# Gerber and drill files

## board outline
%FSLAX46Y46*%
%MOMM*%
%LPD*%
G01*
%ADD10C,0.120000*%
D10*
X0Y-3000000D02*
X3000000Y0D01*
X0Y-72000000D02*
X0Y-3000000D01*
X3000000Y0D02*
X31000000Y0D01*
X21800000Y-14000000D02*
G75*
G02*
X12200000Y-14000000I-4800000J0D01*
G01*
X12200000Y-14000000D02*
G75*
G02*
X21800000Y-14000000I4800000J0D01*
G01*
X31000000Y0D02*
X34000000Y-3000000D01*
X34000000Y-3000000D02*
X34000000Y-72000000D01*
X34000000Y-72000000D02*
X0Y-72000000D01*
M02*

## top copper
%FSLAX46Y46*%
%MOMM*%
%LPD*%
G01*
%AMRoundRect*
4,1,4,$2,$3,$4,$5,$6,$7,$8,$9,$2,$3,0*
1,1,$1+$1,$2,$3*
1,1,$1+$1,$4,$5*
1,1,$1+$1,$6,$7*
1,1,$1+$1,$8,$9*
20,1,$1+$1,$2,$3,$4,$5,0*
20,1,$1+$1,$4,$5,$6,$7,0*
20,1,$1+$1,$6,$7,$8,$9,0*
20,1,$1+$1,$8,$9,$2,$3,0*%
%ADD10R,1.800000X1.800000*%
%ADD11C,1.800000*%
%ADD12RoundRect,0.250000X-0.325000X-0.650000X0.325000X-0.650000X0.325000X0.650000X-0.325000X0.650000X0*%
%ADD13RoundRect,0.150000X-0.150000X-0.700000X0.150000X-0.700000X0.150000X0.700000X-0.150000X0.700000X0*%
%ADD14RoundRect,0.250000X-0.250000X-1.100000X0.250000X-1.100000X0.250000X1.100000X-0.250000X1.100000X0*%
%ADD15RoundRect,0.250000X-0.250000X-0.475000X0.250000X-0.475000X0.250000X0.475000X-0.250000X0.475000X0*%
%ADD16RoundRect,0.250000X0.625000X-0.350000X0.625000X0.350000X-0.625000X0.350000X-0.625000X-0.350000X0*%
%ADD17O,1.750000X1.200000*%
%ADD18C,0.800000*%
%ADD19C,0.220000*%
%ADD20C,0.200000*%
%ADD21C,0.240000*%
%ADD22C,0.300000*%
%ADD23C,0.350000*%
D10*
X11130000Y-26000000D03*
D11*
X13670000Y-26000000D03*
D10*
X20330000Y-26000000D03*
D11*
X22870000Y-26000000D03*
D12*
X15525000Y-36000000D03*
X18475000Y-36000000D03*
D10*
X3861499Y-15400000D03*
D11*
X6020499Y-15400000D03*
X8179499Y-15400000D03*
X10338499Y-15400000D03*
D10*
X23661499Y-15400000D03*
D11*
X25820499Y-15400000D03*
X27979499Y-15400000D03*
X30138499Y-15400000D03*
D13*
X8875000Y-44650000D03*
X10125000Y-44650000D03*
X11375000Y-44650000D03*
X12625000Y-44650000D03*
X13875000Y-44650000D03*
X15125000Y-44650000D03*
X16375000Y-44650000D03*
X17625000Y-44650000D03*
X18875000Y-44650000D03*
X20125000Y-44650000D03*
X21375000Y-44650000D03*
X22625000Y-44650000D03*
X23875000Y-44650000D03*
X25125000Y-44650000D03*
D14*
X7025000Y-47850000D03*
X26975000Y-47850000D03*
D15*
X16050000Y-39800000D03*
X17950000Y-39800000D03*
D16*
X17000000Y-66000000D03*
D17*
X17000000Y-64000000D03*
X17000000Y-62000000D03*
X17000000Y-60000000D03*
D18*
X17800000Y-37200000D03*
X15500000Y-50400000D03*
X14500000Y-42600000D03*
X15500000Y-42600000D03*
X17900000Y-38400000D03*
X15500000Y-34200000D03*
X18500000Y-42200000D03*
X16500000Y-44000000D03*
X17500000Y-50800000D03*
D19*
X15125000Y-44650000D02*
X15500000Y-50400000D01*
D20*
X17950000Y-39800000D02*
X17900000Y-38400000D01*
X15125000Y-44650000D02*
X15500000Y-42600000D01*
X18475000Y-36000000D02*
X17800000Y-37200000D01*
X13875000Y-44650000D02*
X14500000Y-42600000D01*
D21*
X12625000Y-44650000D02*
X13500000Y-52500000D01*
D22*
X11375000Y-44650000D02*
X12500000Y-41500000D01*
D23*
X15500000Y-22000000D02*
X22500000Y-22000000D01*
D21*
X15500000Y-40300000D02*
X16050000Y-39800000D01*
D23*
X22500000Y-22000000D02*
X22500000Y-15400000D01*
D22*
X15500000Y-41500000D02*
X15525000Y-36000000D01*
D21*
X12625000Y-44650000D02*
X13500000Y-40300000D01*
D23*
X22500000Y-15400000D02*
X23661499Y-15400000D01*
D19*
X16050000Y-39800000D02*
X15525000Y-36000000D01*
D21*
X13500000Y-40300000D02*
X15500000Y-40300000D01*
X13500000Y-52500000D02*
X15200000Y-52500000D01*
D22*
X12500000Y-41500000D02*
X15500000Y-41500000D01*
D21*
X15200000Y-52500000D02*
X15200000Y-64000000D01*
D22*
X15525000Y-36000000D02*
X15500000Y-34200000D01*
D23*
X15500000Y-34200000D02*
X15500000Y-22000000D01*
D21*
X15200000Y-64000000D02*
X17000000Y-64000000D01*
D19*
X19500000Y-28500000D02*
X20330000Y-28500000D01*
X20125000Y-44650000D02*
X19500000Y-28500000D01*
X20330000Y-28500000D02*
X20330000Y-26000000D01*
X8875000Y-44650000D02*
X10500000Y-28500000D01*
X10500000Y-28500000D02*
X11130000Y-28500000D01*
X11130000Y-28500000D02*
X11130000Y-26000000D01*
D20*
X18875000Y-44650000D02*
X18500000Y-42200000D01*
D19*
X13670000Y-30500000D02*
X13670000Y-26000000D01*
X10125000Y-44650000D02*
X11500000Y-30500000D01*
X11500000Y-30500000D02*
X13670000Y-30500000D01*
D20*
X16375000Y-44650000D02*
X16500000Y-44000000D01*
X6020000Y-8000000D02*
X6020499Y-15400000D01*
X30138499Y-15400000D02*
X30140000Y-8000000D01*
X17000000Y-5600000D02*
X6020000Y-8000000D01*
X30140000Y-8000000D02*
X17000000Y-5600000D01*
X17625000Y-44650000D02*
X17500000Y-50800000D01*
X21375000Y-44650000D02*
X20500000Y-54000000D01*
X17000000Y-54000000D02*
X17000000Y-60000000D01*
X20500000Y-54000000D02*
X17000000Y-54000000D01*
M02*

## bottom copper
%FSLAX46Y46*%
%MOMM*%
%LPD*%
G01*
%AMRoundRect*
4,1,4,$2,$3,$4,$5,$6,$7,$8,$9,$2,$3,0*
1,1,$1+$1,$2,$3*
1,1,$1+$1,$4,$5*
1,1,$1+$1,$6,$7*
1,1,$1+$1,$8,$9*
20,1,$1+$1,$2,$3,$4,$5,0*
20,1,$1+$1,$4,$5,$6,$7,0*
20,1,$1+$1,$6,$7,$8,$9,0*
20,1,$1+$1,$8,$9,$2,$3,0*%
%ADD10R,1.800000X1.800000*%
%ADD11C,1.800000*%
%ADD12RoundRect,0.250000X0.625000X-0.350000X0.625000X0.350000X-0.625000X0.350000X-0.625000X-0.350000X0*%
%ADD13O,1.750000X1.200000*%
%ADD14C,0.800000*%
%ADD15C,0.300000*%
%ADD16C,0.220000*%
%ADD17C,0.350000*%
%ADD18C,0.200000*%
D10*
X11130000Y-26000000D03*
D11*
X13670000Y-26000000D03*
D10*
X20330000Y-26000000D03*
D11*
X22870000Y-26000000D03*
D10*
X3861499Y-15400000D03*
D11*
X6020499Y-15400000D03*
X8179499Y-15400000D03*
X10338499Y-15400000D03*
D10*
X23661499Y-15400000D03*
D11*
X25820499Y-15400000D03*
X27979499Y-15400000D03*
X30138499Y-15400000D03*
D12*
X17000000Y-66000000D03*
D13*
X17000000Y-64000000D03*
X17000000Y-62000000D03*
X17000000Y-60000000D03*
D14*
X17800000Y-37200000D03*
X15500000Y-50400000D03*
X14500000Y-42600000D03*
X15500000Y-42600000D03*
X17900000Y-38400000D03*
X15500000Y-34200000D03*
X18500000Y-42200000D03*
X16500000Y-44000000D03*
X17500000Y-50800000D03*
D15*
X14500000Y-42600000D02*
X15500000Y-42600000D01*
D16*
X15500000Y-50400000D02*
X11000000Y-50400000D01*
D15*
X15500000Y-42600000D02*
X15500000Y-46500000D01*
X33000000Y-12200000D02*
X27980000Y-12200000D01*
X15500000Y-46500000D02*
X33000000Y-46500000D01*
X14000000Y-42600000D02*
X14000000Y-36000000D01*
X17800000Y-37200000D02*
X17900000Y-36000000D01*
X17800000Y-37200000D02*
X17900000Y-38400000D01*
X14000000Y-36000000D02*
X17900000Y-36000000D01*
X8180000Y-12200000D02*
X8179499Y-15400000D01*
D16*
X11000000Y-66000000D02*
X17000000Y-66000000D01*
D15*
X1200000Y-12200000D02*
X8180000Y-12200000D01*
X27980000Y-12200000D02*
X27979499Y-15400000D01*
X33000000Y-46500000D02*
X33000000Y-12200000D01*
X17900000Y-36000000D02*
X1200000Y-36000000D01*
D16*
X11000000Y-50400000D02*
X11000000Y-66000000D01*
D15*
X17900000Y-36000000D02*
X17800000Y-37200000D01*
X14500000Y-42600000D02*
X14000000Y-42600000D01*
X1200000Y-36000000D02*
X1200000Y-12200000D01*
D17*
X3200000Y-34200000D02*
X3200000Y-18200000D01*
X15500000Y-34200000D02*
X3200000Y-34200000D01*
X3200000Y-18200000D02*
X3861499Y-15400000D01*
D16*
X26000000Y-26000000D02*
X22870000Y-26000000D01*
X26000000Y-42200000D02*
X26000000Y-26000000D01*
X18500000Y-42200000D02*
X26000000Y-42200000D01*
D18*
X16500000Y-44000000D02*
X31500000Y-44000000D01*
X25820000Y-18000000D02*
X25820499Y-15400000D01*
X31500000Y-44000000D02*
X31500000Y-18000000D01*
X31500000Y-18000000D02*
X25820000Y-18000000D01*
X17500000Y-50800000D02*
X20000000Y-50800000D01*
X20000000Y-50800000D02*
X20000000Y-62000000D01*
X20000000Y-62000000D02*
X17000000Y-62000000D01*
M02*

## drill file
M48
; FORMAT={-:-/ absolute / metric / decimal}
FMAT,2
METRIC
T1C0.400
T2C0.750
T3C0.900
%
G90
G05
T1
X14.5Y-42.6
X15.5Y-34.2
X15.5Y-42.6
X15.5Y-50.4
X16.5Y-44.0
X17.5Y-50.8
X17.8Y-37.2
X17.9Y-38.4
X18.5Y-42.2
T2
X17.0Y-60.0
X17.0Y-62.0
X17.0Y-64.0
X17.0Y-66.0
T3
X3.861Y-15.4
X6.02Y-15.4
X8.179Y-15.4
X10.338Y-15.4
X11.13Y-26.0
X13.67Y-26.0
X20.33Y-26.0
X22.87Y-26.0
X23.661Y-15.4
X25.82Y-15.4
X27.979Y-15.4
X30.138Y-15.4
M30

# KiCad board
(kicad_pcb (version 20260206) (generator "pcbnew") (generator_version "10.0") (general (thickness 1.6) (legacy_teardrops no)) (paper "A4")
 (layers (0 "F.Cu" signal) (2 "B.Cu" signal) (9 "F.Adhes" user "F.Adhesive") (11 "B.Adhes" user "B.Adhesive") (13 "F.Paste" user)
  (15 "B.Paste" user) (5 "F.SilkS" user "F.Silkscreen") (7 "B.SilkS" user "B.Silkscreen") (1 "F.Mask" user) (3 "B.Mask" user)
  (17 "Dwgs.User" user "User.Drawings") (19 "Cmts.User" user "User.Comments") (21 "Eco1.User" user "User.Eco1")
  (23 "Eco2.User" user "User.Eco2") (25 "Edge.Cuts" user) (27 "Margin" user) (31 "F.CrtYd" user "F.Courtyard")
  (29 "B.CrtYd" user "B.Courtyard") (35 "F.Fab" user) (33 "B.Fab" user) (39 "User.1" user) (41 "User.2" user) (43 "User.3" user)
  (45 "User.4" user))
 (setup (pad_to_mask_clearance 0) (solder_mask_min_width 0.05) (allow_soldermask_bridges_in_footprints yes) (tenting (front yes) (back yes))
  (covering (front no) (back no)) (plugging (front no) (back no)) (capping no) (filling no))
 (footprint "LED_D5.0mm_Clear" (layer "F.Cu") (at 11.13 26)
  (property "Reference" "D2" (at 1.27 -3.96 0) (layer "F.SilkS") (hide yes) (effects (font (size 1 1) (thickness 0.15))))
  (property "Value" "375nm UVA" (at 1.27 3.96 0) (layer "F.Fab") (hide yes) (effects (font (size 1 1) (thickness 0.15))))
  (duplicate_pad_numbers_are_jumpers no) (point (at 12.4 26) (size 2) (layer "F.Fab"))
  (pad "1" thru_hole rect (at 0 0) (size 1.8 1.8) (drill 0.9) (layers "*.Cu" "*.Mask") (remove_unused_layers no) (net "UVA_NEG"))
  (pad "2" thru_hole circle (at 2.54 0) (size 1.8 1.8) (drill 0.9) (layers "*.Cu" "*.Mask") (remove_unused_layers no) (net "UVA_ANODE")))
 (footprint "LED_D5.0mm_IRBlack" (layer "F.Cu") (at 20.33 26)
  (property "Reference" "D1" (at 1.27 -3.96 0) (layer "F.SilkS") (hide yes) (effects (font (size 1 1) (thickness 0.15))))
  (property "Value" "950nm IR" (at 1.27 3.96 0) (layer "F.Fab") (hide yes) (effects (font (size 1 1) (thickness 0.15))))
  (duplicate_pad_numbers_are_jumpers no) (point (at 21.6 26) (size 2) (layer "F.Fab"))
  (pad "1" thru_hole rect (at 0 0) (size 1.8 1.8) (drill 0.9) (layers "*.Cu" "*.Mask") (remove_unused_layers no) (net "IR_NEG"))
  (pad "2" thru_hole circle (at 2.54 0) (size 1.8 1.8) (drill 0.9) (layers "*.Cu" "*.Mask") (remove_unused_layers no) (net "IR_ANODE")))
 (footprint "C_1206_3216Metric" (layer "F.Cu") (at 17 36)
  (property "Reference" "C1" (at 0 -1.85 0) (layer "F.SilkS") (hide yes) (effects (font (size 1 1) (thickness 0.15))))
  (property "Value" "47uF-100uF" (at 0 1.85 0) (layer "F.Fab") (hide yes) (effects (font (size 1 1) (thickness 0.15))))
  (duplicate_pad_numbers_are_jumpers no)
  (pad "1" smd roundrect (at -1.475 0) (size 1.15 1.8) (layers "F.Cu" "F.Mask" "F.Paste") (roundrect_rratio 0.217391) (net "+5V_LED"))
  (pad "2" smd roundrect (at 1.475 0) (size 1.15 1.8) (layers "F.Cu" "F.Mask" "F.Paste") (roundrect_rratio 0.217391) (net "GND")))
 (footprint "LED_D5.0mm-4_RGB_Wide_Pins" (layer "F.Cu") (at 3.861499 15.4)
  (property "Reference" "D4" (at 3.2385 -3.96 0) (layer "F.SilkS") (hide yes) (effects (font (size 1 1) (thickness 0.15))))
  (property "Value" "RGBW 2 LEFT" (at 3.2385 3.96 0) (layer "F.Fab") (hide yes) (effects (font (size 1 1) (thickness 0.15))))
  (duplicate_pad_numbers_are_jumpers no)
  (pad "1" thru_hole rect (at 0 0) (size 1.8 1.8) (drill 0.9) (layers "*.Cu" "*.Mask") (remove_unused_layers no) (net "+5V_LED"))
  (pad "2" thru_hole circle (at 2.159 0) (size 1.8 1.8) (drill 0.9) (layers "*.Cu" "*.Mask") (remove_unused_layers no) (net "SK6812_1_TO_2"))
  (pad "3" thru_hole circle (at 4.318 0) (size 1.8 1.8) (drill 0.9) (layers "*.Cu" "*.Mask") (remove_unused_layers no) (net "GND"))
  (pad "4" thru_hole circle (at 6.477 0) (size 1.8 1.8) (drill 0.9) (layers "*.Cu" "*.Mask") (remove_unused_layers no)))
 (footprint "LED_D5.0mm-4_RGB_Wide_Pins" (layer "F.Cu") (at 23.661499 15.4)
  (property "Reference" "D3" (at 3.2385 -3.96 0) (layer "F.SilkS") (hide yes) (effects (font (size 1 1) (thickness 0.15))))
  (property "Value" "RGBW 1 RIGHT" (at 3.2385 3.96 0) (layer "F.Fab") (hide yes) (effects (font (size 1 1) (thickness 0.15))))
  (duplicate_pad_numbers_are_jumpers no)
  (pad "1" thru_hole rect (at 0 0) (size 1.8 1.8) (drill 0.9) (layers "*.Cu" "*.Mask") (remove_unused_layers no) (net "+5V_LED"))
  (pad "2" thru_hole circle (at 2.159 0) (size 1.8 1.8) (drill 0.9) (layers "*.Cu" "*.Mask") (remove_unused_layers no) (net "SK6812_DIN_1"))
  (pad "3" thru_hole circle (at 4.318 0) (size 1.8 1.8) (drill 0.9) (layers "*.Cu" "*.Mask") (remove_unused_layers no) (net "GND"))
  (pad "4" thru_hole circle (at 6.477 0) (size 1.8 1.8) (drill 0.9) (layers "*.Cu" "*.Mask") (remove_unused_layers no) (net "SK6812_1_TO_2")))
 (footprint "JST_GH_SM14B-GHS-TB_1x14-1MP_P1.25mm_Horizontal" (layer "F.Cu") (at 17 46.5)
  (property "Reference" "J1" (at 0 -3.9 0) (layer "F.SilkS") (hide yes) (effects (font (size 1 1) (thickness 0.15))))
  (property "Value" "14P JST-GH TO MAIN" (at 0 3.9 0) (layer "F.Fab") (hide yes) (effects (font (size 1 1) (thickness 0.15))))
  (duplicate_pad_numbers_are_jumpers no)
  (pad "1" smd roundrect (at -8.125 -1.85) (size 0.6 1.7) (layers "F.Cu" "F.Mask" "F.Paste") (roundrect_rratio 0.25) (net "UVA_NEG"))
  (pad "2" smd roundrect (at -6.875 -1.85) (size 0.6 1.7) (layers "F.Cu" "F.Mask" "F.Paste") (roundrect_rratio 0.25) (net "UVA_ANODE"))
  (pad "3" smd roundrect (at -5.625 -1.85) (size 0.6 1.7) (layers "F.Cu" "F.Mask" "F.Paste") (roundrect_rratio 0.25) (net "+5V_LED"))
  (pad "4" smd roundrect (at -4.375 -1.85) (size 0.6 1.7) (layers "F.Cu" "F.Mask" "F.Paste") (roundrect_rratio 0.25) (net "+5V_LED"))
  (pad "5" smd roundrect (at -3.125 -1.85) (size 0.6 1.7) (layers "F.Cu" "F.Mask" "F.Paste") (roundrect_rratio 0.25) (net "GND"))
  (pad "6" smd roundrect (at -1.875 -1.85) (size 0.6 1.7) (layers "F.Cu" "F.Mask" "F.Paste") (roundrect_rratio 0.25) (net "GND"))
  (pad "7" smd roundrect (at -0.625 -1.85) (size 0.6 1.7) (layers "F.Cu" "F.Mask" "F.Paste") (roundrect_rratio 0.25) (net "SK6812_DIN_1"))
  (pad "8" smd roundrect (at 0.625 -1.85) (size 0.6 1.7) (layers "F.Cu" "F.Mask" "F.Paste") (roundrect_rratio 0.25) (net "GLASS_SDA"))
  (pad "9" smd roundrect (at 1.875 -1.85) (size 0.6 1.7) (layers "F.Cu" "F.Mask" "F.Paste") (roundrect_rratio 0.25) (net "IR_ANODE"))
  (pad "10" smd roundrect (at 3.125 -1.85) (size 0.6 1.7) (layers "F.Cu" "F.Mask" "F.Paste") (roundrect_rratio 0.25) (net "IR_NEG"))
  (pad "11" smd roundrect (at 4.375 -1.85) (size 0.6 1.7) (layers "F.Cu" "F.Mask" "F.Paste") (roundrect_rratio 0.25) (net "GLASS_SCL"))
  (pad "12" smd roundrect (at 5.625 -1.85) (size 0.6 1.7) (layers "F.Cu" "F.Mask" "F.Paste") (roundrect_rratio 0.25))
  (pad "13" smd roundrect (at 6.875 -1.85) (size 0.6 1.7) (layers "F.Cu" "F.Mask" "F.Paste") (roundrect_rratio 0.25))
  (pad "14" smd roundrect (at 8.125 -1.85) (size 0.6 1.7) (layers "F.Cu" "F.Mask" "F.Paste") (roundrect_rratio 0.25))
  (pad "MP" smd roundrect (at -9.975 1.35) (size 1 2.7) (layers "F.Cu" "F.Mask" "F.Paste") (roundrect_rratio 0.25))
  (pad "MP" smd roundrect (at 9.975 1.35) (size 1 2.7) (layers "F.Cu" "F.Mask" "F.Paste") (roundrect_rratio 0.25)))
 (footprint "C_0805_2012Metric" (layer "F.Cu") (at 17 39.8)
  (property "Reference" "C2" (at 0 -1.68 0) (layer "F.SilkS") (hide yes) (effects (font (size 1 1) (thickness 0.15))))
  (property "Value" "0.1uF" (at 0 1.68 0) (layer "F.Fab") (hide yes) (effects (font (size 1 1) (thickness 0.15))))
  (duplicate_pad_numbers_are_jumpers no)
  (pad "1" smd roundrect (at -0.95 0) (size 1 1.45) (layers "F.Cu" "F.Mask" "F.Paste") (roundrect_rratio 0.25) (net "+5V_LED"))
  (pad "2" smd roundrect (at 0.95 0) (size 1 1.45) (layers "F.Cu" "F.Mask" "F.Paste") (roundrect_rratio 0.25) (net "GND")))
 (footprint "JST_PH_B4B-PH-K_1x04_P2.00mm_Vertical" (layer "F.Cu") (at 17 66 90)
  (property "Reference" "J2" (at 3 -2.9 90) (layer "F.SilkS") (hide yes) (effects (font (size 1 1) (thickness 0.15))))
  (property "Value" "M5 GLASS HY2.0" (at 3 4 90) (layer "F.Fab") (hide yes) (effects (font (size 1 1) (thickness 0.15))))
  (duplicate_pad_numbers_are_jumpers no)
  (pad "1" thru_hole roundrect (at 0 0 90) (size 1.2 1.75) (drill 0.75) (layers "*.Cu" "*.Mask") (remove_unused_layers no)
   (roundrect_rratio 0.208333) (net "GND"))
  (pad "2" thru_hole oval (at 2 0 90) (size 1.2 1.75) (drill 0.75) (layers "*.Cu" "*.Mask") (remove_unused_layers no) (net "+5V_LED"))
  (pad "3" thru_hole oval (at 4 0 90) (size 1.2 1.75) (drill 0.75) (layers "*.Cu" "*.Mask") (remove_unused_layers no) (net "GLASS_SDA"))
  (pad "4" thru_hole oval (at 6 0 90) (size 1.2 1.75) (drill 0.75) (layers "*.Cu" "*.Mask") (remove_unused_layers no) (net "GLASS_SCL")))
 (gr_line (start 0 3) (end 3 0) (stroke (width 0.12) (type default)) (layer "Edge.Cuts"))
 (gr_line (start 0 72) (end 0 3) (stroke (width 0.12) (type default)) (layer "Edge.Cuts"))
 (gr_line (start 3 0) (end 31 0) (stroke (width 0.12) (type default)) (layer "Edge.Cuts"))
 (gr_circle (center 17 14) (end 21.8 14) (stroke (width 0.12) (type default)) (fill no) (layer "Edge.Cuts"))
 (gr_line (start 31 0) (end 34 3) (stroke (width 0.12) (type default)) (layer "Edge.Cuts"))
 (gr_line (start 34 3) (end 34 72) (stroke (width 0.12) (type default)) (layer "Edge.Cuts"))
 (gr_line (start 34 72) (end 0 72) (stroke (width 0.12) (type default)) (layer "Edge.Cuts"))
 (segment (start 15.125 44.65) (end 15.5 50.4) (width 0.22) (layer "F.Cu") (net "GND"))
 (segment (start 17.95 39.8) (end 17.9 38.4) (width 0.2) (layer "F.Cu") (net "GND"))
 (segment (start 15.125 44.65) (end 15.5 42.6) (width 0.2) (layer "F.Cu") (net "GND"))
 (segment (start 18.475 36) (end 17.8 37.2) (width 0.2) (layer "F.Cu") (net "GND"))
 (segment (start 13.875 44.65) (end 14.5 42.6) (width 0.2) (layer "F.Cu") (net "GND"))
 (via (at 17.8 37.2) (size 0.8) (drill 0.4) (layers "F.Cu" "B.Cu") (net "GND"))
 (via (at 15.5 50.4) (size 0.8) (drill 0.4) (layers "F.Cu" "B.Cu") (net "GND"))
 (via (at 14.5 42.6) (size 0.8) (drill 0.4) (layers "F.Cu" "B.Cu") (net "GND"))
 (via (at 15.5 42.6) (size 0.8) (drill 0.4) (layers "F.Cu" "B.Cu") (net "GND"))
 (via (at 17.9 38.4) (size 0.8) (drill 0.4) (layers "F.Cu" "B.Cu") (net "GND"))
 (segment (start 14.5 42.6) (end 15.5 42.6) (width 0.3) (layer "B.Cu") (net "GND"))
 (segment (start 15.5 50.4) (end 11 50.4) (width 0.22) (layer "B.Cu") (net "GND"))
 (segment (start 15.5 42.6) (end 15.5 46.5) (width 0.3) (layer "B.Cu") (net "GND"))
 (segment (start 33 12.2) (end 27.98 12.2) (width 0.3) (layer "B.Cu") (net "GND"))
 (segment (start 15.5 46.5) (end 33 46.5) (width 0.3) (layer "B.Cu") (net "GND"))
 (segment (start 14 42.6) (end 14 36) (width 0.3) (layer "B.Cu") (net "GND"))
 (segment (start 17.8 37.2) (end 17.9 36) (width 0.3) (layer "B.Cu") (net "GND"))
 (segment (start 17.8 37.2) (end 17.9 38.4) (width 0.3) (layer "B.Cu") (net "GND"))
 (segment (start 14 36) (end 17.9 36) (width 0.3) (layer "B.Cu") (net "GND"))
 (segment (start 8.18 12.2) (end 8.179499 15.4) (width 0.3) (layer "B.Cu") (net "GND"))
 (segment (start 11 66) (end 17 66) (width 0.22) (layer "B.Cu") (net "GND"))
 (segment (start 1.2 12.2) (end 8.18 12.2) (width 0.3) (layer "B.Cu") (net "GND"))
 (segment (start 27.98 12.2) (end 27.979499 15.4) (width 0.3) (layer "B.Cu") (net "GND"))
 (segment (start 33 46.5) (end 33 12.2) (width 0.3) (layer "B.Cu") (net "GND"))
 (segment (start 17.9 36) (end 1.2 36) (width 0.3) (layer "B.Cu") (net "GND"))
 (segment (start 11 50.4) (end 11 66) (width 0.22) (layer "B.Cu") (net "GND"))
 (segment (start 17.9 36) (end 17.8 37.2) (width 0.3) (layer "B.Cu") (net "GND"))
 (segment (start 14.5 42.6) (end 14 42.6) (width 0.3) (layer "B.Cu") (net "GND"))
 (segment (start 1.2 36) (end 1.2 12.2) (width 0.3) (layer "B.Cu") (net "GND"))
 (segment (start 12.625 44.65) (end 13.5 52.5) (width 0.24) (layer "F.Cu") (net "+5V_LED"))
 (segment (start 11.375 44.65) (end 12.5 41.5) (width 0.3) (layer "F.Cu") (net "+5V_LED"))
 (segment (start 15.5 22) (end 22.5 22) (width 0.35) (layer "F.Cu") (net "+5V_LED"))
 (segment (start 15.5 40.3) (end 16.05 39.8) (width 0.24) (layer "F.Cu") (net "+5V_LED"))
 (segment (start 22.5 22) (end 22.5 15.4) (width 0.35) (layer "F.Cu") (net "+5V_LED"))
 (segment (start 15.5 41.5) (end 15.525 36) (width 0.3) (layer "F.Cu") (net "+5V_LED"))
 (segment (start 12.625 44.65) (end 13.5 40.3) (width 0.24) (layer "F.Cu") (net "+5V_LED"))
 (segment (start 22.5 15.4) (end 23.661499 15.4) (width 0.35) (layer "F.Cu") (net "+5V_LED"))
 (segment (start 16.05 39.8) (end 15.525 36) (width 0.22) (layer "F.Cu") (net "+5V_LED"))
 (segment (start 13.5 40.3) (end 15.5 40.3) (width 0.24) (layer "F.Cu") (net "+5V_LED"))
 (segment (start 13.5 52.5) (end 15.2 52.5) (width 0.24) (layer "F.Cu") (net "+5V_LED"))
 (segment (start 12.5 41.5) (end 15.5 41.5) (width 0.3) (layer "F.Cu") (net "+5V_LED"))
 (segment (start 15.2 52.5) (end 15.2 64) (width 0.24) (layer "F.Cu") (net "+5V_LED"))
 (segment (start 15.525 36) (end 15.5 34.2) (width 0.3) (layer "F.Cu") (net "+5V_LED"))
 (segment (start 15.5 34.2) (end 15.5 22) (width 0.35) (layer "F.Cu") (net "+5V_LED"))
 (segment (start 15.2 64) (end 17 64) (width 0.24) (layer "F.Cu") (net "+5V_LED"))
 (via (at 15.5 34.2) (size 0.8) (drill 0.4) (layers "F.Cu" "B.Cu") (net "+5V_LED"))
 (segment (start 3.2 34.2) (end 3.2 18.2) (width 0.35) (layer "B.Cu") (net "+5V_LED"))
 (segment (start 15.5 34.2) (end 3.2 34.2) (width 0.35) (layer "B.Cu") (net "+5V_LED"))
 (segment (start 3.2 18.2) (end 3.861499 15.4) (width 0.35) (layer "B.Cu") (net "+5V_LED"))
 (segment (start 19.5 28.5) (end 20.33 28.5) (width 0.22) (layer "F.Cu") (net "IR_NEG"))
 (segment (start 20.125 44.65) (end 19.5 28.5) (width 0.22) (layer "F.Cu") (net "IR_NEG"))
 (segment (start 20.33 28.5) (end 20.33 26) (width 0.22) (layer "F.Cu") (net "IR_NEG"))
 (segment (start 8.875 44.65) (end 10.5 28.5) (width 0.22) (layer "F.Cu") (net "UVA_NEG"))
 (segment (start 10.5 28.5) (end 11.13 28.5) (width 0.22) (layer "F.Cu") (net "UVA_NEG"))
 (segment (start 11.13 28.5) (end 11.13 26) (width 0.22) (layer "F.Cu") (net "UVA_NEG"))
 (segment (start 18.875 44.65) (end 18.5 42.2) (width 0.2) (layer "F.Cu") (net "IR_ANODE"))
 (via (at 18.5 42.2) (size 0.8) (drill 0.4) (layers "F.Cu" "B.Cu") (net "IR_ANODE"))
 (segment (start 26 26) (end 22.87 26) (width 0.22) (layer "B.Cu") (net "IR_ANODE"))
 (segment (start 26 42.2) (end 26 26) (width 0.22) (layer "B.Cu") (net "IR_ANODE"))
 (segment (start 18.5 42.2) (end 26 42.2) (width 0.22) (layer "B.Cu") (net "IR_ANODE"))
 (segment (start 13.67 30.5) (end 13.67 26) (width 0.22) (layer "F.Cu") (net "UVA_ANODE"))
 (segment (start 10.125 44.65) (end 11.5 30.5) (width 0.22) (layer "F.Cu") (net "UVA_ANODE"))
 (segment (start 11.5 30.5) (end 13.67 30.5) (width 0.22) (layer "F.Cu") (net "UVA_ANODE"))
 (segment (start 16.375 44.65) (end 16.5 44) (width 0.2) (layer "F.Cu") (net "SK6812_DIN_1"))
 (via (at 16.5 44) (size 0.8) (drill 0.4) (layers "F.Cu" "B.Cu") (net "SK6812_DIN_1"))
 (segment (start 16.5 44) (end 31.5 44) (width 0.2) (layer "B.Cu") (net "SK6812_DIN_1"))
 (segment (start 25.82 18) (end 25.820499 15.4) (width 0.2) (layer "B.Cu") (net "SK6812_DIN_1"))
 (segment (start 31.5 44) (end 31.5 18) (width 0.2) (layer "B.Cu") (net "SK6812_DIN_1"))
 (segment (start 31.5 18) (end 25.82 18) (width 0.2) (layer "B.Cu") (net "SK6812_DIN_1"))
 (segment (start 6.02 8) (end 6.020499 15.4) (width 0.2) (layer "F.Cu") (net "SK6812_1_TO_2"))
 (segment (start 30.138499 15.4) (end 30.14 8) (width 0.2) (layer "F.Cu") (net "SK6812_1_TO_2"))
 (segment (start 17 5.6) (end 6.02 8) (width 0.2) (layer "F.Cu") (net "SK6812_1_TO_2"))
 (segment (start 30.14 8) (end 17 5.6) (width 0.2) (layer "F.Cu") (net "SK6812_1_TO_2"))
 (segment (start 17.625 44.65) (end 17.5 50.8) (width 0.2) (layer "F.Cu") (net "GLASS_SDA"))
 (via (at 17.5 50.8) (size 0.8) (drill 0.4) (layers "F.Cu" "B.Cu") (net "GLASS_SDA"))
 (segment (start 17.5 50.8) (end 20 50.8) (width 0.2) (layer "B.Cu") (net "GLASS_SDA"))
 (segment (start 20 50.8) (end 20 62) (width 0.2) (layer "B.Cu") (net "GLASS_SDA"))
 (segment (start 20 62) (end 17 62) (width 0.2) (layer "B.Cu") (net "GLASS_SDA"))
 (segment (start 21.375 44.65) (end 20.5 54) (width 0.2) (layer "F.Cu") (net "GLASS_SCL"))
 (segment (start 17 54) (end 17 60) (width 0.2) (layer "F.Cu") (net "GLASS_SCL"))
 (segment (start 20.5 54) (end 17 54) (width 0.2) (layer "F.Cu") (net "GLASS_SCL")))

